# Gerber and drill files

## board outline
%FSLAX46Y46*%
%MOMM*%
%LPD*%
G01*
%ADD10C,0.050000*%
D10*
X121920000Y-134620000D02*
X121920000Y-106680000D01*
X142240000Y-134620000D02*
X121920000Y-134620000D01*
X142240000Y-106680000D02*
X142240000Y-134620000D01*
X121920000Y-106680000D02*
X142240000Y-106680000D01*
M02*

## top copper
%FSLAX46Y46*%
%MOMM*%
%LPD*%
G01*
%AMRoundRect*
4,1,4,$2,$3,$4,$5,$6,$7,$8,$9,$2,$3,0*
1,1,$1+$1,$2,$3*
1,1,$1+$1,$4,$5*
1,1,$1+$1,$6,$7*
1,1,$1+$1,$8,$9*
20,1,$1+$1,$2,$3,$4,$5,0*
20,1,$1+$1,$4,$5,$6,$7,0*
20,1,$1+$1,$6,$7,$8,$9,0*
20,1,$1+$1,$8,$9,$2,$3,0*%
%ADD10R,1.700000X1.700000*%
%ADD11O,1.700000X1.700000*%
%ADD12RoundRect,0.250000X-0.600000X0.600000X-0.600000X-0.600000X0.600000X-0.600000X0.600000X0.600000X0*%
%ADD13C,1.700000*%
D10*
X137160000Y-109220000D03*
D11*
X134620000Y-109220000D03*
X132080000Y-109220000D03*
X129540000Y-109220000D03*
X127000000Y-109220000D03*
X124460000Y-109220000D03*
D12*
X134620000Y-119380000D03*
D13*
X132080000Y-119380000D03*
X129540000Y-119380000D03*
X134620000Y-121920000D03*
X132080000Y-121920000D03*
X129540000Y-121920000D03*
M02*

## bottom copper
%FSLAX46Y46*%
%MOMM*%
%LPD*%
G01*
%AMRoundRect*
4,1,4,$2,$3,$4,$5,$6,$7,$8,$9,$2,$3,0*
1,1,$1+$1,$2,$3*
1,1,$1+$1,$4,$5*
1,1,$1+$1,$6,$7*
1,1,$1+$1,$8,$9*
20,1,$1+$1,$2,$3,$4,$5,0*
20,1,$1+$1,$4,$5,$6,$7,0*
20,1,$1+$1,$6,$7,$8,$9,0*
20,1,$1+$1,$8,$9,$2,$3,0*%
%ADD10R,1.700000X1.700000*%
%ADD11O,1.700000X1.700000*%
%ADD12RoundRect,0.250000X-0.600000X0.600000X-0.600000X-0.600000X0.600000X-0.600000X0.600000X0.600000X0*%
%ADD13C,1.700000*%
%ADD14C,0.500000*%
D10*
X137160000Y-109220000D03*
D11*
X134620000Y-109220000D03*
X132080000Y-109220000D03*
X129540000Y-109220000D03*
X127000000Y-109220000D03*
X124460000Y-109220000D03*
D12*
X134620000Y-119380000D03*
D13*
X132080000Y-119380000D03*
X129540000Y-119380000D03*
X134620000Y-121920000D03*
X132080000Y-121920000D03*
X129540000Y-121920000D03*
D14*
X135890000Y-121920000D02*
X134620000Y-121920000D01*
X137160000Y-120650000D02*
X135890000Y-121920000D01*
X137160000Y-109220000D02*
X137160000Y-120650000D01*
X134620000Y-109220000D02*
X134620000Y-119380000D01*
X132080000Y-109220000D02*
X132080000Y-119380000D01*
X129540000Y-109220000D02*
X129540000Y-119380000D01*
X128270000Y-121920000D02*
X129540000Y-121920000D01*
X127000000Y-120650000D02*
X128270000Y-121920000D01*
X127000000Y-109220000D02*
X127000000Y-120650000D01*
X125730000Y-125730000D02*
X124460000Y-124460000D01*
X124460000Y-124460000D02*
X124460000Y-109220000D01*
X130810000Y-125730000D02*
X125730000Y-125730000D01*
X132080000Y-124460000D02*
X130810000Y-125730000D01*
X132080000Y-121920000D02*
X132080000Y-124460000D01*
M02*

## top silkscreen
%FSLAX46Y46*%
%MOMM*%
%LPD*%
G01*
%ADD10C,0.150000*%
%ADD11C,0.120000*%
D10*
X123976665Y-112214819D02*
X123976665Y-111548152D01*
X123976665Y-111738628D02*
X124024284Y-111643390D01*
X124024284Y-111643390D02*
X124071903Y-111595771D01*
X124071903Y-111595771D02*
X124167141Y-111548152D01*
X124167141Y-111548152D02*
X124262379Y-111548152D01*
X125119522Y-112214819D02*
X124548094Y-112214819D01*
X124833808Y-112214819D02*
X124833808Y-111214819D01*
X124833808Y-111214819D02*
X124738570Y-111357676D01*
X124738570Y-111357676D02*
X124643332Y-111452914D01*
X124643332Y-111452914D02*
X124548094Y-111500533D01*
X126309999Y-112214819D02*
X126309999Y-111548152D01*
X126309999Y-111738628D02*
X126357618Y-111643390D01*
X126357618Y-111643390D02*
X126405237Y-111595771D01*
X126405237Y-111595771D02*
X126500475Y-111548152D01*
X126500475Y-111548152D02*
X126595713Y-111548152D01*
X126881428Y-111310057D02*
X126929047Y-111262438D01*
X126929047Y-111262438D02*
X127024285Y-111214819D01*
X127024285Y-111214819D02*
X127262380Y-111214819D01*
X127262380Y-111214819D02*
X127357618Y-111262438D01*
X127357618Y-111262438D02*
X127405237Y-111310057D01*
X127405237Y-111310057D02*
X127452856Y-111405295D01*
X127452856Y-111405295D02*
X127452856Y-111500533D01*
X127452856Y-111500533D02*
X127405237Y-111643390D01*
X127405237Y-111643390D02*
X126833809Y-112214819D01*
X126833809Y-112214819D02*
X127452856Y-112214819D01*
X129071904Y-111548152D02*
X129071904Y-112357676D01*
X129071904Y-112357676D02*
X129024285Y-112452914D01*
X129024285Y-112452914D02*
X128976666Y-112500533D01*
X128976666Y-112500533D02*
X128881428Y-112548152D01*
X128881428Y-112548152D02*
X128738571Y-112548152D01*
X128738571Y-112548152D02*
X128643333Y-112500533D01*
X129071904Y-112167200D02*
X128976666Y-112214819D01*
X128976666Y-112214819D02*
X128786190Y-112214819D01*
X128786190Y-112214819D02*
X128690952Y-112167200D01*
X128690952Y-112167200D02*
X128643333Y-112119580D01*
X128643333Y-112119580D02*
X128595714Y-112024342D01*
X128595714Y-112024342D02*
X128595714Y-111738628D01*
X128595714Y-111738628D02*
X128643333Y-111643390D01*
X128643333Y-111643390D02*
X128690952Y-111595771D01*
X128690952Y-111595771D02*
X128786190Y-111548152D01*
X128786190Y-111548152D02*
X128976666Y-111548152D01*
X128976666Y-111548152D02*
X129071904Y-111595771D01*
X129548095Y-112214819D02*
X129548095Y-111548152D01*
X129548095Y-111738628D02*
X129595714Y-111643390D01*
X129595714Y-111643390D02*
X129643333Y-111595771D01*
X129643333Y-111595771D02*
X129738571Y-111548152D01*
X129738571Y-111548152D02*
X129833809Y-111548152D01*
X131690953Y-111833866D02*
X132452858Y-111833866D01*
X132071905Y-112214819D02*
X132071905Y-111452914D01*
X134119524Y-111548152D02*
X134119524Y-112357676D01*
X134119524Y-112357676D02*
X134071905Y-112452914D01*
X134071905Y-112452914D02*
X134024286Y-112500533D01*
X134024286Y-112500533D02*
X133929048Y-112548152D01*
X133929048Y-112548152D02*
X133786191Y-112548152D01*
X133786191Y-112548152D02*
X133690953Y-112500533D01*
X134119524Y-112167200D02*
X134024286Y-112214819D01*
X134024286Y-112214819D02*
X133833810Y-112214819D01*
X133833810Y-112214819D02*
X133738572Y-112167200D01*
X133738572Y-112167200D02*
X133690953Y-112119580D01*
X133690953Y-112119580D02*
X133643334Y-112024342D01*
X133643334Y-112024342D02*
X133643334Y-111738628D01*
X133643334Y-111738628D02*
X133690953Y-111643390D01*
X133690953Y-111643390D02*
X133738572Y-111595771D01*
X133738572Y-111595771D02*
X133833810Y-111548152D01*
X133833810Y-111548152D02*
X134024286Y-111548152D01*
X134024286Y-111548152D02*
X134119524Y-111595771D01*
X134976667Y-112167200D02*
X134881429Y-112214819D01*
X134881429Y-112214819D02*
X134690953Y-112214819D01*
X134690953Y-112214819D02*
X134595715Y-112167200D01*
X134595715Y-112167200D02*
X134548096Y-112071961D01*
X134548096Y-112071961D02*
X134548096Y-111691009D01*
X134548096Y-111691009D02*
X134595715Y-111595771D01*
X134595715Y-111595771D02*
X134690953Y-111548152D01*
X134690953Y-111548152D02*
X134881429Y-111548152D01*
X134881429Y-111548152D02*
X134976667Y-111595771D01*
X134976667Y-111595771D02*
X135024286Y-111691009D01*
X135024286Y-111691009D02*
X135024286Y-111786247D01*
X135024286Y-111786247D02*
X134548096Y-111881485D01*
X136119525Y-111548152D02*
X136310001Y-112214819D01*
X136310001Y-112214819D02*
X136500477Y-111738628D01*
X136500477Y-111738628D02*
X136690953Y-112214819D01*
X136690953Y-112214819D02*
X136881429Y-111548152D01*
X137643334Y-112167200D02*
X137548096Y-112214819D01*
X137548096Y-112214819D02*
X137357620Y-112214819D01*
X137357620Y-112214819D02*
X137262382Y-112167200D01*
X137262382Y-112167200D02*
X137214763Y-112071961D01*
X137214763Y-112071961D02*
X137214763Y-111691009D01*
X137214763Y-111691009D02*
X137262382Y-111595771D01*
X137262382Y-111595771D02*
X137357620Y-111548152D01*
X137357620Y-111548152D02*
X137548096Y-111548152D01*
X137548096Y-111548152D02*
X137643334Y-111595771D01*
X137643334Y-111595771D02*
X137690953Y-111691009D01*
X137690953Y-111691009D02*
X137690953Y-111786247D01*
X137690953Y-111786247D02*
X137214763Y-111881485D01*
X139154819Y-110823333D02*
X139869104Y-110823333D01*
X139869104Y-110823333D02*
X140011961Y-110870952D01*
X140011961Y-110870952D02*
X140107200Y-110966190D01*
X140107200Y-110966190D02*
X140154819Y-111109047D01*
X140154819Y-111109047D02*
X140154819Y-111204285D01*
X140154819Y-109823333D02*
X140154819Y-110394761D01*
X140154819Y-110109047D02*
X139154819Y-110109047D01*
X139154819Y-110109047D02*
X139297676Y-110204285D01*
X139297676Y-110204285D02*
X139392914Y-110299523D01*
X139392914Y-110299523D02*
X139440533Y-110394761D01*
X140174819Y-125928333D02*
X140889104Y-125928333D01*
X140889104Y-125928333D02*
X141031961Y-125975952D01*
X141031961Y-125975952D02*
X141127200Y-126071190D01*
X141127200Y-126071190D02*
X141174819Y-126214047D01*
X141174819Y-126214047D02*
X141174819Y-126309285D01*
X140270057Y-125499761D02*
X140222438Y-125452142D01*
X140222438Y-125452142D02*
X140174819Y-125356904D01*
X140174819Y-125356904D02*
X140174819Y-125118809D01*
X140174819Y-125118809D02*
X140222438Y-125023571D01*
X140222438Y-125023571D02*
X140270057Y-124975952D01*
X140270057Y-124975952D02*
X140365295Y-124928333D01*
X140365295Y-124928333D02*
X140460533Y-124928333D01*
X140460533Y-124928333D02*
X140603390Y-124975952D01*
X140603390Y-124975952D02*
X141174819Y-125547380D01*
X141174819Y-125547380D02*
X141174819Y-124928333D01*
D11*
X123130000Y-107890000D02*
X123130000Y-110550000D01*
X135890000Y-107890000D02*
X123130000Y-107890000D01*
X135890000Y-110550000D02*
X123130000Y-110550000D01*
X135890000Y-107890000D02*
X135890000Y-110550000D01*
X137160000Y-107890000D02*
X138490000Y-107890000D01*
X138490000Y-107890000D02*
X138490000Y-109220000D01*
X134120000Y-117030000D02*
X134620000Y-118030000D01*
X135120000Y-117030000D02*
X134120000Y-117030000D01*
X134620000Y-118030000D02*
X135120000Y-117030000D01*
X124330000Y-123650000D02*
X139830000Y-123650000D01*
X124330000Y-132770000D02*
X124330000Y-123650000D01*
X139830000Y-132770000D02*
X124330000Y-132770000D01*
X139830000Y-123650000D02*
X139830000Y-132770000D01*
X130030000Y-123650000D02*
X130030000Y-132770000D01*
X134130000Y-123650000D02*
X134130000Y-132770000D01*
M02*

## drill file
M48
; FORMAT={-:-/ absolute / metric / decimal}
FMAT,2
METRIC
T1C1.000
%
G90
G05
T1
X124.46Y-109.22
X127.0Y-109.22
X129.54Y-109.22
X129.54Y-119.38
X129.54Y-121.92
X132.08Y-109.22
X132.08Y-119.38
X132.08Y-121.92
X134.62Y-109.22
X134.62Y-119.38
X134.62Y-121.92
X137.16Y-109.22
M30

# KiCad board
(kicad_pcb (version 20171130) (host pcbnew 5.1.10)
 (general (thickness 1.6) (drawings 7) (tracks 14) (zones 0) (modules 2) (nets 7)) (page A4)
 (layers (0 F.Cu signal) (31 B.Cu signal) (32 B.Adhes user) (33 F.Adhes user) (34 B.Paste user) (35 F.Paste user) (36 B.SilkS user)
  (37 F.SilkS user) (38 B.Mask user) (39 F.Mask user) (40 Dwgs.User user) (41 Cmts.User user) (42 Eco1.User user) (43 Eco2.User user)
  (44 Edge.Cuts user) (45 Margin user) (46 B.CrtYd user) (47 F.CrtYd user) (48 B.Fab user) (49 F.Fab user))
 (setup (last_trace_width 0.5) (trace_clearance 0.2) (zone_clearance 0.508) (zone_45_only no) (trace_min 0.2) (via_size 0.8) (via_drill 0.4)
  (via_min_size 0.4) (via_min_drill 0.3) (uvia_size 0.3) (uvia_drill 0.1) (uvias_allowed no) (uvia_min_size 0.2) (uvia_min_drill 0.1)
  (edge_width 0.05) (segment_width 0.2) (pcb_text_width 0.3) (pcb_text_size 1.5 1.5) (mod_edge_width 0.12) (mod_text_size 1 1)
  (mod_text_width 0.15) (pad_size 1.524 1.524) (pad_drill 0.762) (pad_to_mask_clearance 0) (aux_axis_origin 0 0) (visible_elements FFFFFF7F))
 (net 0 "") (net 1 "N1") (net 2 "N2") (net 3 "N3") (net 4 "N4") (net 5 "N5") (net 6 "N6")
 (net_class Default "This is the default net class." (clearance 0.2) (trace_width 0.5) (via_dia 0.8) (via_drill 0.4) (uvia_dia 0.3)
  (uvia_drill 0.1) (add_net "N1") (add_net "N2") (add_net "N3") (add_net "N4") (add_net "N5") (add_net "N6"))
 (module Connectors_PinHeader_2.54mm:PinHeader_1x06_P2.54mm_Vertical (layer F.Cu) (at 137.16 109.22 270)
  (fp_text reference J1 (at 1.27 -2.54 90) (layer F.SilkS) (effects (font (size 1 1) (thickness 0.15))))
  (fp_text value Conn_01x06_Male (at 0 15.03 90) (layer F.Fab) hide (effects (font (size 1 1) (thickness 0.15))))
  (fp_line (start -1.33 14.03) (end 1.33 14.03) (layer F.SilkS) (width 0.12))
  (fp_line (start -1.33 1.27) (end -1.33 14.03) (layer F.SilkS) (width 0.12))
  (fp_line (start 1.33 1.27) (end 1.33 14.03) (layer F.SilkS) (width 0.12))
  (fp_line (start -1.33 1.27) (end 1.33 1.27) (layer F.SilkS) (width 0.12))
  (fp_line (start -1.33 0) (end -1.33 -1.33) (layer F.SilkS) (width 0.12))
  (fp_line (start -1.33 -1.33) (end 0 -1.33) (layer F.SilkS) (width 0.12))
  (pad 1 thru_hole rect (at 0 0 270) (size 1.7 1.7) (drill 1) (layers *.Cu *.Mask) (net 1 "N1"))
  (pad 2 thru_hole oval (at 0 2.54 270) (size 1.7 1.7) (drill 1) (layers *.Cu *.Mask) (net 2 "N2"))
  (pad 3 thru_hole oval (at 0 5.08 270) (size 1.7 1.7) (drill 1) (layers *.Cu *.Mask) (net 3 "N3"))
  (pad 4 thru_hole oval (at 0 7.62 270) (size 1.7 1.7) (drill 1) (layers *.Cu *.Mask) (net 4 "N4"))
  (pad 5 thru_hole oval (at 0 10.16 270) (size 1.7 1.7) (drill 1) (layers *.Cu *.Mask) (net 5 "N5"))
  (pad 6 thru_hole oval (at 0 12.7 270) (size 1.7 1.7) (drill 1) (layers *.Cu *.Mask) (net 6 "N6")))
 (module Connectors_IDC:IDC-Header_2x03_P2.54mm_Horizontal (layer F.Cu) (at 134.62 119.38 270)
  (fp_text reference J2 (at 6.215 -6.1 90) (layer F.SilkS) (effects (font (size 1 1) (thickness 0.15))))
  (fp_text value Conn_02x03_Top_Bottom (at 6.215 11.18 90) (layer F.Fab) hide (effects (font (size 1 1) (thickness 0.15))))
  (fp_line (start -2.35 0.5) (end -1.35 0) (layer F.SilkS) (width 0.12))
  (fp_line (start -2.35 -0.5) (end -2.35 0.5) (layer F.SilkS) (width 0.12))
  (fp_line (start -1.35 0) (end -2.35 -0.5) (layer F.SilkS) (width 0.12))
  (fp_line (start 4.27 10.29) (end 4.27 -5.21) (layer F.SilkS) (width 0.12))
  (fp_line (start 13.39 10.29) (end 4.27 10.29) (layer F.SilkS) (width 0.12))
  (fp_line (start 13.39 -5.21) (end 13.39 10.29) (layer F.SilkS) (width 0.12))
  (fp_line (start 4.27 -5.21) (end 13.39 -5.21) (layer F.SilkS) (width 0.12))
  (fp_line (start 4.27 4.59) (end 13.39 4.59) (layer F.SilkS) (width 0.12))
  (fp_line (start 4.27 0.49) (end 13.39 0.49) (layer F.SilkS) (width 0.12))
  (pad 1 thru_hole roundrect (at 0 0 270) (size 1.7 1.7) (drill 1) (layers *.Cu *.Mask) (roundrect_rratio 0.1470588235294118) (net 2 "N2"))
  (pad 3 thru_hole circle (at 0 2.54 270) (size 1.7 1.7) (drill 1) (layers *.Cu *.Mask) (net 3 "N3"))
  (pad 5 thru_hole circle (at 0 5.08 270) (size 1.7 1.7) (drill 1) (layers *.Cu *.Mask) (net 4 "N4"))
  (pad 2 thru_hole circle (at 2.54 0 270) (size 1.7 1.7) (drill 1) (layers *.Cu *.Mask) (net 1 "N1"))
  (pad 4 thru_hole circle (at 2.54 2.54 270) (size 1.7 1.7) (drill 1) (layers *.Cu *.Mask) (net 6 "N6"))
  (pad 6 thru_hole circle (at 2.54 5.08 270) (size 1.7 1.7) (drill 1) (layers *.Cu *.Mask) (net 5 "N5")))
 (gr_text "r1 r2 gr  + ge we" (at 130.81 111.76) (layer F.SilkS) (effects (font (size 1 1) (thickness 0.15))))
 (gr_line (start 121.92 134.62) (end 121.92 106.68) (layer Edge.Cuts) (width 0.05))
 (gr_line (start 142.24 134.62) (end 121.92 134.62) (layer Edge.Cuts) (width 0.05))
 (gr_line (start 142.24 106.68) (end 142.24 134.62) (layer Edge.Cuts) (width 0.05))
 (gr_line (start 121.92 106.68) (end 142.24 106.68) (layer Edge.Cuts) (width 0.05))
 (segment (start 135.89 121.92) (end 134.62 121.92) (width 0.5) (layer B.Cu) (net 1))
 (segment (start 137.16 120.65) (end 135.89 121.92) (width 0.5) (layer B.Cu) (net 1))
 (segment (start 137.16 109.22) (end 137.16 120.65) (width 0.5) (layer B.Cu) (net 1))
 (segment (start 134.62 109.22) (end 134.62 119.38) (width 0.5) (layer B.Cu) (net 2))
 (segment (start 132.08 109.22) (end 132.08 119.38) (width 0.5) (layer B.Cu) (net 3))
 (segment (start 129.54 109.22) (end 129.54 119.38) (width 0.5) (layer B.Cu) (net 4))
 (segment (start 128.27 121.92) (end 129.54 121.92) (width 0.5) (layer B.Cu) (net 5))
 (segment (start 127 120.65) (end 128.27 121.92) (width 0.5) (layer B.Cu) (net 5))
 (segment (start 127 109.22) (end 127 120.65) (width 0.5) (layer B.Cu) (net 5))
 (segment (start 125.73 125.73) (end 124.46 124.46) (width 0.5) (layer B.Cu) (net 6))
 (segment (start 124.46 124.46) (end 124.46 109.22) (width 0.5) (layer B.Cu) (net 6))
 (segment (start 130.81 125.73) (end 125.73 125.73) (width 0.5) (layer B.Cu) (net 6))
 (segment (start 132.08 124.46) (end 130.81 125.73) (width 0.5) (layer B.Cu) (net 6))
 (segment (start 132.08 121.92) (end 132.08 124.46) (width 0.5) (layer B.Cu) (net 6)))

